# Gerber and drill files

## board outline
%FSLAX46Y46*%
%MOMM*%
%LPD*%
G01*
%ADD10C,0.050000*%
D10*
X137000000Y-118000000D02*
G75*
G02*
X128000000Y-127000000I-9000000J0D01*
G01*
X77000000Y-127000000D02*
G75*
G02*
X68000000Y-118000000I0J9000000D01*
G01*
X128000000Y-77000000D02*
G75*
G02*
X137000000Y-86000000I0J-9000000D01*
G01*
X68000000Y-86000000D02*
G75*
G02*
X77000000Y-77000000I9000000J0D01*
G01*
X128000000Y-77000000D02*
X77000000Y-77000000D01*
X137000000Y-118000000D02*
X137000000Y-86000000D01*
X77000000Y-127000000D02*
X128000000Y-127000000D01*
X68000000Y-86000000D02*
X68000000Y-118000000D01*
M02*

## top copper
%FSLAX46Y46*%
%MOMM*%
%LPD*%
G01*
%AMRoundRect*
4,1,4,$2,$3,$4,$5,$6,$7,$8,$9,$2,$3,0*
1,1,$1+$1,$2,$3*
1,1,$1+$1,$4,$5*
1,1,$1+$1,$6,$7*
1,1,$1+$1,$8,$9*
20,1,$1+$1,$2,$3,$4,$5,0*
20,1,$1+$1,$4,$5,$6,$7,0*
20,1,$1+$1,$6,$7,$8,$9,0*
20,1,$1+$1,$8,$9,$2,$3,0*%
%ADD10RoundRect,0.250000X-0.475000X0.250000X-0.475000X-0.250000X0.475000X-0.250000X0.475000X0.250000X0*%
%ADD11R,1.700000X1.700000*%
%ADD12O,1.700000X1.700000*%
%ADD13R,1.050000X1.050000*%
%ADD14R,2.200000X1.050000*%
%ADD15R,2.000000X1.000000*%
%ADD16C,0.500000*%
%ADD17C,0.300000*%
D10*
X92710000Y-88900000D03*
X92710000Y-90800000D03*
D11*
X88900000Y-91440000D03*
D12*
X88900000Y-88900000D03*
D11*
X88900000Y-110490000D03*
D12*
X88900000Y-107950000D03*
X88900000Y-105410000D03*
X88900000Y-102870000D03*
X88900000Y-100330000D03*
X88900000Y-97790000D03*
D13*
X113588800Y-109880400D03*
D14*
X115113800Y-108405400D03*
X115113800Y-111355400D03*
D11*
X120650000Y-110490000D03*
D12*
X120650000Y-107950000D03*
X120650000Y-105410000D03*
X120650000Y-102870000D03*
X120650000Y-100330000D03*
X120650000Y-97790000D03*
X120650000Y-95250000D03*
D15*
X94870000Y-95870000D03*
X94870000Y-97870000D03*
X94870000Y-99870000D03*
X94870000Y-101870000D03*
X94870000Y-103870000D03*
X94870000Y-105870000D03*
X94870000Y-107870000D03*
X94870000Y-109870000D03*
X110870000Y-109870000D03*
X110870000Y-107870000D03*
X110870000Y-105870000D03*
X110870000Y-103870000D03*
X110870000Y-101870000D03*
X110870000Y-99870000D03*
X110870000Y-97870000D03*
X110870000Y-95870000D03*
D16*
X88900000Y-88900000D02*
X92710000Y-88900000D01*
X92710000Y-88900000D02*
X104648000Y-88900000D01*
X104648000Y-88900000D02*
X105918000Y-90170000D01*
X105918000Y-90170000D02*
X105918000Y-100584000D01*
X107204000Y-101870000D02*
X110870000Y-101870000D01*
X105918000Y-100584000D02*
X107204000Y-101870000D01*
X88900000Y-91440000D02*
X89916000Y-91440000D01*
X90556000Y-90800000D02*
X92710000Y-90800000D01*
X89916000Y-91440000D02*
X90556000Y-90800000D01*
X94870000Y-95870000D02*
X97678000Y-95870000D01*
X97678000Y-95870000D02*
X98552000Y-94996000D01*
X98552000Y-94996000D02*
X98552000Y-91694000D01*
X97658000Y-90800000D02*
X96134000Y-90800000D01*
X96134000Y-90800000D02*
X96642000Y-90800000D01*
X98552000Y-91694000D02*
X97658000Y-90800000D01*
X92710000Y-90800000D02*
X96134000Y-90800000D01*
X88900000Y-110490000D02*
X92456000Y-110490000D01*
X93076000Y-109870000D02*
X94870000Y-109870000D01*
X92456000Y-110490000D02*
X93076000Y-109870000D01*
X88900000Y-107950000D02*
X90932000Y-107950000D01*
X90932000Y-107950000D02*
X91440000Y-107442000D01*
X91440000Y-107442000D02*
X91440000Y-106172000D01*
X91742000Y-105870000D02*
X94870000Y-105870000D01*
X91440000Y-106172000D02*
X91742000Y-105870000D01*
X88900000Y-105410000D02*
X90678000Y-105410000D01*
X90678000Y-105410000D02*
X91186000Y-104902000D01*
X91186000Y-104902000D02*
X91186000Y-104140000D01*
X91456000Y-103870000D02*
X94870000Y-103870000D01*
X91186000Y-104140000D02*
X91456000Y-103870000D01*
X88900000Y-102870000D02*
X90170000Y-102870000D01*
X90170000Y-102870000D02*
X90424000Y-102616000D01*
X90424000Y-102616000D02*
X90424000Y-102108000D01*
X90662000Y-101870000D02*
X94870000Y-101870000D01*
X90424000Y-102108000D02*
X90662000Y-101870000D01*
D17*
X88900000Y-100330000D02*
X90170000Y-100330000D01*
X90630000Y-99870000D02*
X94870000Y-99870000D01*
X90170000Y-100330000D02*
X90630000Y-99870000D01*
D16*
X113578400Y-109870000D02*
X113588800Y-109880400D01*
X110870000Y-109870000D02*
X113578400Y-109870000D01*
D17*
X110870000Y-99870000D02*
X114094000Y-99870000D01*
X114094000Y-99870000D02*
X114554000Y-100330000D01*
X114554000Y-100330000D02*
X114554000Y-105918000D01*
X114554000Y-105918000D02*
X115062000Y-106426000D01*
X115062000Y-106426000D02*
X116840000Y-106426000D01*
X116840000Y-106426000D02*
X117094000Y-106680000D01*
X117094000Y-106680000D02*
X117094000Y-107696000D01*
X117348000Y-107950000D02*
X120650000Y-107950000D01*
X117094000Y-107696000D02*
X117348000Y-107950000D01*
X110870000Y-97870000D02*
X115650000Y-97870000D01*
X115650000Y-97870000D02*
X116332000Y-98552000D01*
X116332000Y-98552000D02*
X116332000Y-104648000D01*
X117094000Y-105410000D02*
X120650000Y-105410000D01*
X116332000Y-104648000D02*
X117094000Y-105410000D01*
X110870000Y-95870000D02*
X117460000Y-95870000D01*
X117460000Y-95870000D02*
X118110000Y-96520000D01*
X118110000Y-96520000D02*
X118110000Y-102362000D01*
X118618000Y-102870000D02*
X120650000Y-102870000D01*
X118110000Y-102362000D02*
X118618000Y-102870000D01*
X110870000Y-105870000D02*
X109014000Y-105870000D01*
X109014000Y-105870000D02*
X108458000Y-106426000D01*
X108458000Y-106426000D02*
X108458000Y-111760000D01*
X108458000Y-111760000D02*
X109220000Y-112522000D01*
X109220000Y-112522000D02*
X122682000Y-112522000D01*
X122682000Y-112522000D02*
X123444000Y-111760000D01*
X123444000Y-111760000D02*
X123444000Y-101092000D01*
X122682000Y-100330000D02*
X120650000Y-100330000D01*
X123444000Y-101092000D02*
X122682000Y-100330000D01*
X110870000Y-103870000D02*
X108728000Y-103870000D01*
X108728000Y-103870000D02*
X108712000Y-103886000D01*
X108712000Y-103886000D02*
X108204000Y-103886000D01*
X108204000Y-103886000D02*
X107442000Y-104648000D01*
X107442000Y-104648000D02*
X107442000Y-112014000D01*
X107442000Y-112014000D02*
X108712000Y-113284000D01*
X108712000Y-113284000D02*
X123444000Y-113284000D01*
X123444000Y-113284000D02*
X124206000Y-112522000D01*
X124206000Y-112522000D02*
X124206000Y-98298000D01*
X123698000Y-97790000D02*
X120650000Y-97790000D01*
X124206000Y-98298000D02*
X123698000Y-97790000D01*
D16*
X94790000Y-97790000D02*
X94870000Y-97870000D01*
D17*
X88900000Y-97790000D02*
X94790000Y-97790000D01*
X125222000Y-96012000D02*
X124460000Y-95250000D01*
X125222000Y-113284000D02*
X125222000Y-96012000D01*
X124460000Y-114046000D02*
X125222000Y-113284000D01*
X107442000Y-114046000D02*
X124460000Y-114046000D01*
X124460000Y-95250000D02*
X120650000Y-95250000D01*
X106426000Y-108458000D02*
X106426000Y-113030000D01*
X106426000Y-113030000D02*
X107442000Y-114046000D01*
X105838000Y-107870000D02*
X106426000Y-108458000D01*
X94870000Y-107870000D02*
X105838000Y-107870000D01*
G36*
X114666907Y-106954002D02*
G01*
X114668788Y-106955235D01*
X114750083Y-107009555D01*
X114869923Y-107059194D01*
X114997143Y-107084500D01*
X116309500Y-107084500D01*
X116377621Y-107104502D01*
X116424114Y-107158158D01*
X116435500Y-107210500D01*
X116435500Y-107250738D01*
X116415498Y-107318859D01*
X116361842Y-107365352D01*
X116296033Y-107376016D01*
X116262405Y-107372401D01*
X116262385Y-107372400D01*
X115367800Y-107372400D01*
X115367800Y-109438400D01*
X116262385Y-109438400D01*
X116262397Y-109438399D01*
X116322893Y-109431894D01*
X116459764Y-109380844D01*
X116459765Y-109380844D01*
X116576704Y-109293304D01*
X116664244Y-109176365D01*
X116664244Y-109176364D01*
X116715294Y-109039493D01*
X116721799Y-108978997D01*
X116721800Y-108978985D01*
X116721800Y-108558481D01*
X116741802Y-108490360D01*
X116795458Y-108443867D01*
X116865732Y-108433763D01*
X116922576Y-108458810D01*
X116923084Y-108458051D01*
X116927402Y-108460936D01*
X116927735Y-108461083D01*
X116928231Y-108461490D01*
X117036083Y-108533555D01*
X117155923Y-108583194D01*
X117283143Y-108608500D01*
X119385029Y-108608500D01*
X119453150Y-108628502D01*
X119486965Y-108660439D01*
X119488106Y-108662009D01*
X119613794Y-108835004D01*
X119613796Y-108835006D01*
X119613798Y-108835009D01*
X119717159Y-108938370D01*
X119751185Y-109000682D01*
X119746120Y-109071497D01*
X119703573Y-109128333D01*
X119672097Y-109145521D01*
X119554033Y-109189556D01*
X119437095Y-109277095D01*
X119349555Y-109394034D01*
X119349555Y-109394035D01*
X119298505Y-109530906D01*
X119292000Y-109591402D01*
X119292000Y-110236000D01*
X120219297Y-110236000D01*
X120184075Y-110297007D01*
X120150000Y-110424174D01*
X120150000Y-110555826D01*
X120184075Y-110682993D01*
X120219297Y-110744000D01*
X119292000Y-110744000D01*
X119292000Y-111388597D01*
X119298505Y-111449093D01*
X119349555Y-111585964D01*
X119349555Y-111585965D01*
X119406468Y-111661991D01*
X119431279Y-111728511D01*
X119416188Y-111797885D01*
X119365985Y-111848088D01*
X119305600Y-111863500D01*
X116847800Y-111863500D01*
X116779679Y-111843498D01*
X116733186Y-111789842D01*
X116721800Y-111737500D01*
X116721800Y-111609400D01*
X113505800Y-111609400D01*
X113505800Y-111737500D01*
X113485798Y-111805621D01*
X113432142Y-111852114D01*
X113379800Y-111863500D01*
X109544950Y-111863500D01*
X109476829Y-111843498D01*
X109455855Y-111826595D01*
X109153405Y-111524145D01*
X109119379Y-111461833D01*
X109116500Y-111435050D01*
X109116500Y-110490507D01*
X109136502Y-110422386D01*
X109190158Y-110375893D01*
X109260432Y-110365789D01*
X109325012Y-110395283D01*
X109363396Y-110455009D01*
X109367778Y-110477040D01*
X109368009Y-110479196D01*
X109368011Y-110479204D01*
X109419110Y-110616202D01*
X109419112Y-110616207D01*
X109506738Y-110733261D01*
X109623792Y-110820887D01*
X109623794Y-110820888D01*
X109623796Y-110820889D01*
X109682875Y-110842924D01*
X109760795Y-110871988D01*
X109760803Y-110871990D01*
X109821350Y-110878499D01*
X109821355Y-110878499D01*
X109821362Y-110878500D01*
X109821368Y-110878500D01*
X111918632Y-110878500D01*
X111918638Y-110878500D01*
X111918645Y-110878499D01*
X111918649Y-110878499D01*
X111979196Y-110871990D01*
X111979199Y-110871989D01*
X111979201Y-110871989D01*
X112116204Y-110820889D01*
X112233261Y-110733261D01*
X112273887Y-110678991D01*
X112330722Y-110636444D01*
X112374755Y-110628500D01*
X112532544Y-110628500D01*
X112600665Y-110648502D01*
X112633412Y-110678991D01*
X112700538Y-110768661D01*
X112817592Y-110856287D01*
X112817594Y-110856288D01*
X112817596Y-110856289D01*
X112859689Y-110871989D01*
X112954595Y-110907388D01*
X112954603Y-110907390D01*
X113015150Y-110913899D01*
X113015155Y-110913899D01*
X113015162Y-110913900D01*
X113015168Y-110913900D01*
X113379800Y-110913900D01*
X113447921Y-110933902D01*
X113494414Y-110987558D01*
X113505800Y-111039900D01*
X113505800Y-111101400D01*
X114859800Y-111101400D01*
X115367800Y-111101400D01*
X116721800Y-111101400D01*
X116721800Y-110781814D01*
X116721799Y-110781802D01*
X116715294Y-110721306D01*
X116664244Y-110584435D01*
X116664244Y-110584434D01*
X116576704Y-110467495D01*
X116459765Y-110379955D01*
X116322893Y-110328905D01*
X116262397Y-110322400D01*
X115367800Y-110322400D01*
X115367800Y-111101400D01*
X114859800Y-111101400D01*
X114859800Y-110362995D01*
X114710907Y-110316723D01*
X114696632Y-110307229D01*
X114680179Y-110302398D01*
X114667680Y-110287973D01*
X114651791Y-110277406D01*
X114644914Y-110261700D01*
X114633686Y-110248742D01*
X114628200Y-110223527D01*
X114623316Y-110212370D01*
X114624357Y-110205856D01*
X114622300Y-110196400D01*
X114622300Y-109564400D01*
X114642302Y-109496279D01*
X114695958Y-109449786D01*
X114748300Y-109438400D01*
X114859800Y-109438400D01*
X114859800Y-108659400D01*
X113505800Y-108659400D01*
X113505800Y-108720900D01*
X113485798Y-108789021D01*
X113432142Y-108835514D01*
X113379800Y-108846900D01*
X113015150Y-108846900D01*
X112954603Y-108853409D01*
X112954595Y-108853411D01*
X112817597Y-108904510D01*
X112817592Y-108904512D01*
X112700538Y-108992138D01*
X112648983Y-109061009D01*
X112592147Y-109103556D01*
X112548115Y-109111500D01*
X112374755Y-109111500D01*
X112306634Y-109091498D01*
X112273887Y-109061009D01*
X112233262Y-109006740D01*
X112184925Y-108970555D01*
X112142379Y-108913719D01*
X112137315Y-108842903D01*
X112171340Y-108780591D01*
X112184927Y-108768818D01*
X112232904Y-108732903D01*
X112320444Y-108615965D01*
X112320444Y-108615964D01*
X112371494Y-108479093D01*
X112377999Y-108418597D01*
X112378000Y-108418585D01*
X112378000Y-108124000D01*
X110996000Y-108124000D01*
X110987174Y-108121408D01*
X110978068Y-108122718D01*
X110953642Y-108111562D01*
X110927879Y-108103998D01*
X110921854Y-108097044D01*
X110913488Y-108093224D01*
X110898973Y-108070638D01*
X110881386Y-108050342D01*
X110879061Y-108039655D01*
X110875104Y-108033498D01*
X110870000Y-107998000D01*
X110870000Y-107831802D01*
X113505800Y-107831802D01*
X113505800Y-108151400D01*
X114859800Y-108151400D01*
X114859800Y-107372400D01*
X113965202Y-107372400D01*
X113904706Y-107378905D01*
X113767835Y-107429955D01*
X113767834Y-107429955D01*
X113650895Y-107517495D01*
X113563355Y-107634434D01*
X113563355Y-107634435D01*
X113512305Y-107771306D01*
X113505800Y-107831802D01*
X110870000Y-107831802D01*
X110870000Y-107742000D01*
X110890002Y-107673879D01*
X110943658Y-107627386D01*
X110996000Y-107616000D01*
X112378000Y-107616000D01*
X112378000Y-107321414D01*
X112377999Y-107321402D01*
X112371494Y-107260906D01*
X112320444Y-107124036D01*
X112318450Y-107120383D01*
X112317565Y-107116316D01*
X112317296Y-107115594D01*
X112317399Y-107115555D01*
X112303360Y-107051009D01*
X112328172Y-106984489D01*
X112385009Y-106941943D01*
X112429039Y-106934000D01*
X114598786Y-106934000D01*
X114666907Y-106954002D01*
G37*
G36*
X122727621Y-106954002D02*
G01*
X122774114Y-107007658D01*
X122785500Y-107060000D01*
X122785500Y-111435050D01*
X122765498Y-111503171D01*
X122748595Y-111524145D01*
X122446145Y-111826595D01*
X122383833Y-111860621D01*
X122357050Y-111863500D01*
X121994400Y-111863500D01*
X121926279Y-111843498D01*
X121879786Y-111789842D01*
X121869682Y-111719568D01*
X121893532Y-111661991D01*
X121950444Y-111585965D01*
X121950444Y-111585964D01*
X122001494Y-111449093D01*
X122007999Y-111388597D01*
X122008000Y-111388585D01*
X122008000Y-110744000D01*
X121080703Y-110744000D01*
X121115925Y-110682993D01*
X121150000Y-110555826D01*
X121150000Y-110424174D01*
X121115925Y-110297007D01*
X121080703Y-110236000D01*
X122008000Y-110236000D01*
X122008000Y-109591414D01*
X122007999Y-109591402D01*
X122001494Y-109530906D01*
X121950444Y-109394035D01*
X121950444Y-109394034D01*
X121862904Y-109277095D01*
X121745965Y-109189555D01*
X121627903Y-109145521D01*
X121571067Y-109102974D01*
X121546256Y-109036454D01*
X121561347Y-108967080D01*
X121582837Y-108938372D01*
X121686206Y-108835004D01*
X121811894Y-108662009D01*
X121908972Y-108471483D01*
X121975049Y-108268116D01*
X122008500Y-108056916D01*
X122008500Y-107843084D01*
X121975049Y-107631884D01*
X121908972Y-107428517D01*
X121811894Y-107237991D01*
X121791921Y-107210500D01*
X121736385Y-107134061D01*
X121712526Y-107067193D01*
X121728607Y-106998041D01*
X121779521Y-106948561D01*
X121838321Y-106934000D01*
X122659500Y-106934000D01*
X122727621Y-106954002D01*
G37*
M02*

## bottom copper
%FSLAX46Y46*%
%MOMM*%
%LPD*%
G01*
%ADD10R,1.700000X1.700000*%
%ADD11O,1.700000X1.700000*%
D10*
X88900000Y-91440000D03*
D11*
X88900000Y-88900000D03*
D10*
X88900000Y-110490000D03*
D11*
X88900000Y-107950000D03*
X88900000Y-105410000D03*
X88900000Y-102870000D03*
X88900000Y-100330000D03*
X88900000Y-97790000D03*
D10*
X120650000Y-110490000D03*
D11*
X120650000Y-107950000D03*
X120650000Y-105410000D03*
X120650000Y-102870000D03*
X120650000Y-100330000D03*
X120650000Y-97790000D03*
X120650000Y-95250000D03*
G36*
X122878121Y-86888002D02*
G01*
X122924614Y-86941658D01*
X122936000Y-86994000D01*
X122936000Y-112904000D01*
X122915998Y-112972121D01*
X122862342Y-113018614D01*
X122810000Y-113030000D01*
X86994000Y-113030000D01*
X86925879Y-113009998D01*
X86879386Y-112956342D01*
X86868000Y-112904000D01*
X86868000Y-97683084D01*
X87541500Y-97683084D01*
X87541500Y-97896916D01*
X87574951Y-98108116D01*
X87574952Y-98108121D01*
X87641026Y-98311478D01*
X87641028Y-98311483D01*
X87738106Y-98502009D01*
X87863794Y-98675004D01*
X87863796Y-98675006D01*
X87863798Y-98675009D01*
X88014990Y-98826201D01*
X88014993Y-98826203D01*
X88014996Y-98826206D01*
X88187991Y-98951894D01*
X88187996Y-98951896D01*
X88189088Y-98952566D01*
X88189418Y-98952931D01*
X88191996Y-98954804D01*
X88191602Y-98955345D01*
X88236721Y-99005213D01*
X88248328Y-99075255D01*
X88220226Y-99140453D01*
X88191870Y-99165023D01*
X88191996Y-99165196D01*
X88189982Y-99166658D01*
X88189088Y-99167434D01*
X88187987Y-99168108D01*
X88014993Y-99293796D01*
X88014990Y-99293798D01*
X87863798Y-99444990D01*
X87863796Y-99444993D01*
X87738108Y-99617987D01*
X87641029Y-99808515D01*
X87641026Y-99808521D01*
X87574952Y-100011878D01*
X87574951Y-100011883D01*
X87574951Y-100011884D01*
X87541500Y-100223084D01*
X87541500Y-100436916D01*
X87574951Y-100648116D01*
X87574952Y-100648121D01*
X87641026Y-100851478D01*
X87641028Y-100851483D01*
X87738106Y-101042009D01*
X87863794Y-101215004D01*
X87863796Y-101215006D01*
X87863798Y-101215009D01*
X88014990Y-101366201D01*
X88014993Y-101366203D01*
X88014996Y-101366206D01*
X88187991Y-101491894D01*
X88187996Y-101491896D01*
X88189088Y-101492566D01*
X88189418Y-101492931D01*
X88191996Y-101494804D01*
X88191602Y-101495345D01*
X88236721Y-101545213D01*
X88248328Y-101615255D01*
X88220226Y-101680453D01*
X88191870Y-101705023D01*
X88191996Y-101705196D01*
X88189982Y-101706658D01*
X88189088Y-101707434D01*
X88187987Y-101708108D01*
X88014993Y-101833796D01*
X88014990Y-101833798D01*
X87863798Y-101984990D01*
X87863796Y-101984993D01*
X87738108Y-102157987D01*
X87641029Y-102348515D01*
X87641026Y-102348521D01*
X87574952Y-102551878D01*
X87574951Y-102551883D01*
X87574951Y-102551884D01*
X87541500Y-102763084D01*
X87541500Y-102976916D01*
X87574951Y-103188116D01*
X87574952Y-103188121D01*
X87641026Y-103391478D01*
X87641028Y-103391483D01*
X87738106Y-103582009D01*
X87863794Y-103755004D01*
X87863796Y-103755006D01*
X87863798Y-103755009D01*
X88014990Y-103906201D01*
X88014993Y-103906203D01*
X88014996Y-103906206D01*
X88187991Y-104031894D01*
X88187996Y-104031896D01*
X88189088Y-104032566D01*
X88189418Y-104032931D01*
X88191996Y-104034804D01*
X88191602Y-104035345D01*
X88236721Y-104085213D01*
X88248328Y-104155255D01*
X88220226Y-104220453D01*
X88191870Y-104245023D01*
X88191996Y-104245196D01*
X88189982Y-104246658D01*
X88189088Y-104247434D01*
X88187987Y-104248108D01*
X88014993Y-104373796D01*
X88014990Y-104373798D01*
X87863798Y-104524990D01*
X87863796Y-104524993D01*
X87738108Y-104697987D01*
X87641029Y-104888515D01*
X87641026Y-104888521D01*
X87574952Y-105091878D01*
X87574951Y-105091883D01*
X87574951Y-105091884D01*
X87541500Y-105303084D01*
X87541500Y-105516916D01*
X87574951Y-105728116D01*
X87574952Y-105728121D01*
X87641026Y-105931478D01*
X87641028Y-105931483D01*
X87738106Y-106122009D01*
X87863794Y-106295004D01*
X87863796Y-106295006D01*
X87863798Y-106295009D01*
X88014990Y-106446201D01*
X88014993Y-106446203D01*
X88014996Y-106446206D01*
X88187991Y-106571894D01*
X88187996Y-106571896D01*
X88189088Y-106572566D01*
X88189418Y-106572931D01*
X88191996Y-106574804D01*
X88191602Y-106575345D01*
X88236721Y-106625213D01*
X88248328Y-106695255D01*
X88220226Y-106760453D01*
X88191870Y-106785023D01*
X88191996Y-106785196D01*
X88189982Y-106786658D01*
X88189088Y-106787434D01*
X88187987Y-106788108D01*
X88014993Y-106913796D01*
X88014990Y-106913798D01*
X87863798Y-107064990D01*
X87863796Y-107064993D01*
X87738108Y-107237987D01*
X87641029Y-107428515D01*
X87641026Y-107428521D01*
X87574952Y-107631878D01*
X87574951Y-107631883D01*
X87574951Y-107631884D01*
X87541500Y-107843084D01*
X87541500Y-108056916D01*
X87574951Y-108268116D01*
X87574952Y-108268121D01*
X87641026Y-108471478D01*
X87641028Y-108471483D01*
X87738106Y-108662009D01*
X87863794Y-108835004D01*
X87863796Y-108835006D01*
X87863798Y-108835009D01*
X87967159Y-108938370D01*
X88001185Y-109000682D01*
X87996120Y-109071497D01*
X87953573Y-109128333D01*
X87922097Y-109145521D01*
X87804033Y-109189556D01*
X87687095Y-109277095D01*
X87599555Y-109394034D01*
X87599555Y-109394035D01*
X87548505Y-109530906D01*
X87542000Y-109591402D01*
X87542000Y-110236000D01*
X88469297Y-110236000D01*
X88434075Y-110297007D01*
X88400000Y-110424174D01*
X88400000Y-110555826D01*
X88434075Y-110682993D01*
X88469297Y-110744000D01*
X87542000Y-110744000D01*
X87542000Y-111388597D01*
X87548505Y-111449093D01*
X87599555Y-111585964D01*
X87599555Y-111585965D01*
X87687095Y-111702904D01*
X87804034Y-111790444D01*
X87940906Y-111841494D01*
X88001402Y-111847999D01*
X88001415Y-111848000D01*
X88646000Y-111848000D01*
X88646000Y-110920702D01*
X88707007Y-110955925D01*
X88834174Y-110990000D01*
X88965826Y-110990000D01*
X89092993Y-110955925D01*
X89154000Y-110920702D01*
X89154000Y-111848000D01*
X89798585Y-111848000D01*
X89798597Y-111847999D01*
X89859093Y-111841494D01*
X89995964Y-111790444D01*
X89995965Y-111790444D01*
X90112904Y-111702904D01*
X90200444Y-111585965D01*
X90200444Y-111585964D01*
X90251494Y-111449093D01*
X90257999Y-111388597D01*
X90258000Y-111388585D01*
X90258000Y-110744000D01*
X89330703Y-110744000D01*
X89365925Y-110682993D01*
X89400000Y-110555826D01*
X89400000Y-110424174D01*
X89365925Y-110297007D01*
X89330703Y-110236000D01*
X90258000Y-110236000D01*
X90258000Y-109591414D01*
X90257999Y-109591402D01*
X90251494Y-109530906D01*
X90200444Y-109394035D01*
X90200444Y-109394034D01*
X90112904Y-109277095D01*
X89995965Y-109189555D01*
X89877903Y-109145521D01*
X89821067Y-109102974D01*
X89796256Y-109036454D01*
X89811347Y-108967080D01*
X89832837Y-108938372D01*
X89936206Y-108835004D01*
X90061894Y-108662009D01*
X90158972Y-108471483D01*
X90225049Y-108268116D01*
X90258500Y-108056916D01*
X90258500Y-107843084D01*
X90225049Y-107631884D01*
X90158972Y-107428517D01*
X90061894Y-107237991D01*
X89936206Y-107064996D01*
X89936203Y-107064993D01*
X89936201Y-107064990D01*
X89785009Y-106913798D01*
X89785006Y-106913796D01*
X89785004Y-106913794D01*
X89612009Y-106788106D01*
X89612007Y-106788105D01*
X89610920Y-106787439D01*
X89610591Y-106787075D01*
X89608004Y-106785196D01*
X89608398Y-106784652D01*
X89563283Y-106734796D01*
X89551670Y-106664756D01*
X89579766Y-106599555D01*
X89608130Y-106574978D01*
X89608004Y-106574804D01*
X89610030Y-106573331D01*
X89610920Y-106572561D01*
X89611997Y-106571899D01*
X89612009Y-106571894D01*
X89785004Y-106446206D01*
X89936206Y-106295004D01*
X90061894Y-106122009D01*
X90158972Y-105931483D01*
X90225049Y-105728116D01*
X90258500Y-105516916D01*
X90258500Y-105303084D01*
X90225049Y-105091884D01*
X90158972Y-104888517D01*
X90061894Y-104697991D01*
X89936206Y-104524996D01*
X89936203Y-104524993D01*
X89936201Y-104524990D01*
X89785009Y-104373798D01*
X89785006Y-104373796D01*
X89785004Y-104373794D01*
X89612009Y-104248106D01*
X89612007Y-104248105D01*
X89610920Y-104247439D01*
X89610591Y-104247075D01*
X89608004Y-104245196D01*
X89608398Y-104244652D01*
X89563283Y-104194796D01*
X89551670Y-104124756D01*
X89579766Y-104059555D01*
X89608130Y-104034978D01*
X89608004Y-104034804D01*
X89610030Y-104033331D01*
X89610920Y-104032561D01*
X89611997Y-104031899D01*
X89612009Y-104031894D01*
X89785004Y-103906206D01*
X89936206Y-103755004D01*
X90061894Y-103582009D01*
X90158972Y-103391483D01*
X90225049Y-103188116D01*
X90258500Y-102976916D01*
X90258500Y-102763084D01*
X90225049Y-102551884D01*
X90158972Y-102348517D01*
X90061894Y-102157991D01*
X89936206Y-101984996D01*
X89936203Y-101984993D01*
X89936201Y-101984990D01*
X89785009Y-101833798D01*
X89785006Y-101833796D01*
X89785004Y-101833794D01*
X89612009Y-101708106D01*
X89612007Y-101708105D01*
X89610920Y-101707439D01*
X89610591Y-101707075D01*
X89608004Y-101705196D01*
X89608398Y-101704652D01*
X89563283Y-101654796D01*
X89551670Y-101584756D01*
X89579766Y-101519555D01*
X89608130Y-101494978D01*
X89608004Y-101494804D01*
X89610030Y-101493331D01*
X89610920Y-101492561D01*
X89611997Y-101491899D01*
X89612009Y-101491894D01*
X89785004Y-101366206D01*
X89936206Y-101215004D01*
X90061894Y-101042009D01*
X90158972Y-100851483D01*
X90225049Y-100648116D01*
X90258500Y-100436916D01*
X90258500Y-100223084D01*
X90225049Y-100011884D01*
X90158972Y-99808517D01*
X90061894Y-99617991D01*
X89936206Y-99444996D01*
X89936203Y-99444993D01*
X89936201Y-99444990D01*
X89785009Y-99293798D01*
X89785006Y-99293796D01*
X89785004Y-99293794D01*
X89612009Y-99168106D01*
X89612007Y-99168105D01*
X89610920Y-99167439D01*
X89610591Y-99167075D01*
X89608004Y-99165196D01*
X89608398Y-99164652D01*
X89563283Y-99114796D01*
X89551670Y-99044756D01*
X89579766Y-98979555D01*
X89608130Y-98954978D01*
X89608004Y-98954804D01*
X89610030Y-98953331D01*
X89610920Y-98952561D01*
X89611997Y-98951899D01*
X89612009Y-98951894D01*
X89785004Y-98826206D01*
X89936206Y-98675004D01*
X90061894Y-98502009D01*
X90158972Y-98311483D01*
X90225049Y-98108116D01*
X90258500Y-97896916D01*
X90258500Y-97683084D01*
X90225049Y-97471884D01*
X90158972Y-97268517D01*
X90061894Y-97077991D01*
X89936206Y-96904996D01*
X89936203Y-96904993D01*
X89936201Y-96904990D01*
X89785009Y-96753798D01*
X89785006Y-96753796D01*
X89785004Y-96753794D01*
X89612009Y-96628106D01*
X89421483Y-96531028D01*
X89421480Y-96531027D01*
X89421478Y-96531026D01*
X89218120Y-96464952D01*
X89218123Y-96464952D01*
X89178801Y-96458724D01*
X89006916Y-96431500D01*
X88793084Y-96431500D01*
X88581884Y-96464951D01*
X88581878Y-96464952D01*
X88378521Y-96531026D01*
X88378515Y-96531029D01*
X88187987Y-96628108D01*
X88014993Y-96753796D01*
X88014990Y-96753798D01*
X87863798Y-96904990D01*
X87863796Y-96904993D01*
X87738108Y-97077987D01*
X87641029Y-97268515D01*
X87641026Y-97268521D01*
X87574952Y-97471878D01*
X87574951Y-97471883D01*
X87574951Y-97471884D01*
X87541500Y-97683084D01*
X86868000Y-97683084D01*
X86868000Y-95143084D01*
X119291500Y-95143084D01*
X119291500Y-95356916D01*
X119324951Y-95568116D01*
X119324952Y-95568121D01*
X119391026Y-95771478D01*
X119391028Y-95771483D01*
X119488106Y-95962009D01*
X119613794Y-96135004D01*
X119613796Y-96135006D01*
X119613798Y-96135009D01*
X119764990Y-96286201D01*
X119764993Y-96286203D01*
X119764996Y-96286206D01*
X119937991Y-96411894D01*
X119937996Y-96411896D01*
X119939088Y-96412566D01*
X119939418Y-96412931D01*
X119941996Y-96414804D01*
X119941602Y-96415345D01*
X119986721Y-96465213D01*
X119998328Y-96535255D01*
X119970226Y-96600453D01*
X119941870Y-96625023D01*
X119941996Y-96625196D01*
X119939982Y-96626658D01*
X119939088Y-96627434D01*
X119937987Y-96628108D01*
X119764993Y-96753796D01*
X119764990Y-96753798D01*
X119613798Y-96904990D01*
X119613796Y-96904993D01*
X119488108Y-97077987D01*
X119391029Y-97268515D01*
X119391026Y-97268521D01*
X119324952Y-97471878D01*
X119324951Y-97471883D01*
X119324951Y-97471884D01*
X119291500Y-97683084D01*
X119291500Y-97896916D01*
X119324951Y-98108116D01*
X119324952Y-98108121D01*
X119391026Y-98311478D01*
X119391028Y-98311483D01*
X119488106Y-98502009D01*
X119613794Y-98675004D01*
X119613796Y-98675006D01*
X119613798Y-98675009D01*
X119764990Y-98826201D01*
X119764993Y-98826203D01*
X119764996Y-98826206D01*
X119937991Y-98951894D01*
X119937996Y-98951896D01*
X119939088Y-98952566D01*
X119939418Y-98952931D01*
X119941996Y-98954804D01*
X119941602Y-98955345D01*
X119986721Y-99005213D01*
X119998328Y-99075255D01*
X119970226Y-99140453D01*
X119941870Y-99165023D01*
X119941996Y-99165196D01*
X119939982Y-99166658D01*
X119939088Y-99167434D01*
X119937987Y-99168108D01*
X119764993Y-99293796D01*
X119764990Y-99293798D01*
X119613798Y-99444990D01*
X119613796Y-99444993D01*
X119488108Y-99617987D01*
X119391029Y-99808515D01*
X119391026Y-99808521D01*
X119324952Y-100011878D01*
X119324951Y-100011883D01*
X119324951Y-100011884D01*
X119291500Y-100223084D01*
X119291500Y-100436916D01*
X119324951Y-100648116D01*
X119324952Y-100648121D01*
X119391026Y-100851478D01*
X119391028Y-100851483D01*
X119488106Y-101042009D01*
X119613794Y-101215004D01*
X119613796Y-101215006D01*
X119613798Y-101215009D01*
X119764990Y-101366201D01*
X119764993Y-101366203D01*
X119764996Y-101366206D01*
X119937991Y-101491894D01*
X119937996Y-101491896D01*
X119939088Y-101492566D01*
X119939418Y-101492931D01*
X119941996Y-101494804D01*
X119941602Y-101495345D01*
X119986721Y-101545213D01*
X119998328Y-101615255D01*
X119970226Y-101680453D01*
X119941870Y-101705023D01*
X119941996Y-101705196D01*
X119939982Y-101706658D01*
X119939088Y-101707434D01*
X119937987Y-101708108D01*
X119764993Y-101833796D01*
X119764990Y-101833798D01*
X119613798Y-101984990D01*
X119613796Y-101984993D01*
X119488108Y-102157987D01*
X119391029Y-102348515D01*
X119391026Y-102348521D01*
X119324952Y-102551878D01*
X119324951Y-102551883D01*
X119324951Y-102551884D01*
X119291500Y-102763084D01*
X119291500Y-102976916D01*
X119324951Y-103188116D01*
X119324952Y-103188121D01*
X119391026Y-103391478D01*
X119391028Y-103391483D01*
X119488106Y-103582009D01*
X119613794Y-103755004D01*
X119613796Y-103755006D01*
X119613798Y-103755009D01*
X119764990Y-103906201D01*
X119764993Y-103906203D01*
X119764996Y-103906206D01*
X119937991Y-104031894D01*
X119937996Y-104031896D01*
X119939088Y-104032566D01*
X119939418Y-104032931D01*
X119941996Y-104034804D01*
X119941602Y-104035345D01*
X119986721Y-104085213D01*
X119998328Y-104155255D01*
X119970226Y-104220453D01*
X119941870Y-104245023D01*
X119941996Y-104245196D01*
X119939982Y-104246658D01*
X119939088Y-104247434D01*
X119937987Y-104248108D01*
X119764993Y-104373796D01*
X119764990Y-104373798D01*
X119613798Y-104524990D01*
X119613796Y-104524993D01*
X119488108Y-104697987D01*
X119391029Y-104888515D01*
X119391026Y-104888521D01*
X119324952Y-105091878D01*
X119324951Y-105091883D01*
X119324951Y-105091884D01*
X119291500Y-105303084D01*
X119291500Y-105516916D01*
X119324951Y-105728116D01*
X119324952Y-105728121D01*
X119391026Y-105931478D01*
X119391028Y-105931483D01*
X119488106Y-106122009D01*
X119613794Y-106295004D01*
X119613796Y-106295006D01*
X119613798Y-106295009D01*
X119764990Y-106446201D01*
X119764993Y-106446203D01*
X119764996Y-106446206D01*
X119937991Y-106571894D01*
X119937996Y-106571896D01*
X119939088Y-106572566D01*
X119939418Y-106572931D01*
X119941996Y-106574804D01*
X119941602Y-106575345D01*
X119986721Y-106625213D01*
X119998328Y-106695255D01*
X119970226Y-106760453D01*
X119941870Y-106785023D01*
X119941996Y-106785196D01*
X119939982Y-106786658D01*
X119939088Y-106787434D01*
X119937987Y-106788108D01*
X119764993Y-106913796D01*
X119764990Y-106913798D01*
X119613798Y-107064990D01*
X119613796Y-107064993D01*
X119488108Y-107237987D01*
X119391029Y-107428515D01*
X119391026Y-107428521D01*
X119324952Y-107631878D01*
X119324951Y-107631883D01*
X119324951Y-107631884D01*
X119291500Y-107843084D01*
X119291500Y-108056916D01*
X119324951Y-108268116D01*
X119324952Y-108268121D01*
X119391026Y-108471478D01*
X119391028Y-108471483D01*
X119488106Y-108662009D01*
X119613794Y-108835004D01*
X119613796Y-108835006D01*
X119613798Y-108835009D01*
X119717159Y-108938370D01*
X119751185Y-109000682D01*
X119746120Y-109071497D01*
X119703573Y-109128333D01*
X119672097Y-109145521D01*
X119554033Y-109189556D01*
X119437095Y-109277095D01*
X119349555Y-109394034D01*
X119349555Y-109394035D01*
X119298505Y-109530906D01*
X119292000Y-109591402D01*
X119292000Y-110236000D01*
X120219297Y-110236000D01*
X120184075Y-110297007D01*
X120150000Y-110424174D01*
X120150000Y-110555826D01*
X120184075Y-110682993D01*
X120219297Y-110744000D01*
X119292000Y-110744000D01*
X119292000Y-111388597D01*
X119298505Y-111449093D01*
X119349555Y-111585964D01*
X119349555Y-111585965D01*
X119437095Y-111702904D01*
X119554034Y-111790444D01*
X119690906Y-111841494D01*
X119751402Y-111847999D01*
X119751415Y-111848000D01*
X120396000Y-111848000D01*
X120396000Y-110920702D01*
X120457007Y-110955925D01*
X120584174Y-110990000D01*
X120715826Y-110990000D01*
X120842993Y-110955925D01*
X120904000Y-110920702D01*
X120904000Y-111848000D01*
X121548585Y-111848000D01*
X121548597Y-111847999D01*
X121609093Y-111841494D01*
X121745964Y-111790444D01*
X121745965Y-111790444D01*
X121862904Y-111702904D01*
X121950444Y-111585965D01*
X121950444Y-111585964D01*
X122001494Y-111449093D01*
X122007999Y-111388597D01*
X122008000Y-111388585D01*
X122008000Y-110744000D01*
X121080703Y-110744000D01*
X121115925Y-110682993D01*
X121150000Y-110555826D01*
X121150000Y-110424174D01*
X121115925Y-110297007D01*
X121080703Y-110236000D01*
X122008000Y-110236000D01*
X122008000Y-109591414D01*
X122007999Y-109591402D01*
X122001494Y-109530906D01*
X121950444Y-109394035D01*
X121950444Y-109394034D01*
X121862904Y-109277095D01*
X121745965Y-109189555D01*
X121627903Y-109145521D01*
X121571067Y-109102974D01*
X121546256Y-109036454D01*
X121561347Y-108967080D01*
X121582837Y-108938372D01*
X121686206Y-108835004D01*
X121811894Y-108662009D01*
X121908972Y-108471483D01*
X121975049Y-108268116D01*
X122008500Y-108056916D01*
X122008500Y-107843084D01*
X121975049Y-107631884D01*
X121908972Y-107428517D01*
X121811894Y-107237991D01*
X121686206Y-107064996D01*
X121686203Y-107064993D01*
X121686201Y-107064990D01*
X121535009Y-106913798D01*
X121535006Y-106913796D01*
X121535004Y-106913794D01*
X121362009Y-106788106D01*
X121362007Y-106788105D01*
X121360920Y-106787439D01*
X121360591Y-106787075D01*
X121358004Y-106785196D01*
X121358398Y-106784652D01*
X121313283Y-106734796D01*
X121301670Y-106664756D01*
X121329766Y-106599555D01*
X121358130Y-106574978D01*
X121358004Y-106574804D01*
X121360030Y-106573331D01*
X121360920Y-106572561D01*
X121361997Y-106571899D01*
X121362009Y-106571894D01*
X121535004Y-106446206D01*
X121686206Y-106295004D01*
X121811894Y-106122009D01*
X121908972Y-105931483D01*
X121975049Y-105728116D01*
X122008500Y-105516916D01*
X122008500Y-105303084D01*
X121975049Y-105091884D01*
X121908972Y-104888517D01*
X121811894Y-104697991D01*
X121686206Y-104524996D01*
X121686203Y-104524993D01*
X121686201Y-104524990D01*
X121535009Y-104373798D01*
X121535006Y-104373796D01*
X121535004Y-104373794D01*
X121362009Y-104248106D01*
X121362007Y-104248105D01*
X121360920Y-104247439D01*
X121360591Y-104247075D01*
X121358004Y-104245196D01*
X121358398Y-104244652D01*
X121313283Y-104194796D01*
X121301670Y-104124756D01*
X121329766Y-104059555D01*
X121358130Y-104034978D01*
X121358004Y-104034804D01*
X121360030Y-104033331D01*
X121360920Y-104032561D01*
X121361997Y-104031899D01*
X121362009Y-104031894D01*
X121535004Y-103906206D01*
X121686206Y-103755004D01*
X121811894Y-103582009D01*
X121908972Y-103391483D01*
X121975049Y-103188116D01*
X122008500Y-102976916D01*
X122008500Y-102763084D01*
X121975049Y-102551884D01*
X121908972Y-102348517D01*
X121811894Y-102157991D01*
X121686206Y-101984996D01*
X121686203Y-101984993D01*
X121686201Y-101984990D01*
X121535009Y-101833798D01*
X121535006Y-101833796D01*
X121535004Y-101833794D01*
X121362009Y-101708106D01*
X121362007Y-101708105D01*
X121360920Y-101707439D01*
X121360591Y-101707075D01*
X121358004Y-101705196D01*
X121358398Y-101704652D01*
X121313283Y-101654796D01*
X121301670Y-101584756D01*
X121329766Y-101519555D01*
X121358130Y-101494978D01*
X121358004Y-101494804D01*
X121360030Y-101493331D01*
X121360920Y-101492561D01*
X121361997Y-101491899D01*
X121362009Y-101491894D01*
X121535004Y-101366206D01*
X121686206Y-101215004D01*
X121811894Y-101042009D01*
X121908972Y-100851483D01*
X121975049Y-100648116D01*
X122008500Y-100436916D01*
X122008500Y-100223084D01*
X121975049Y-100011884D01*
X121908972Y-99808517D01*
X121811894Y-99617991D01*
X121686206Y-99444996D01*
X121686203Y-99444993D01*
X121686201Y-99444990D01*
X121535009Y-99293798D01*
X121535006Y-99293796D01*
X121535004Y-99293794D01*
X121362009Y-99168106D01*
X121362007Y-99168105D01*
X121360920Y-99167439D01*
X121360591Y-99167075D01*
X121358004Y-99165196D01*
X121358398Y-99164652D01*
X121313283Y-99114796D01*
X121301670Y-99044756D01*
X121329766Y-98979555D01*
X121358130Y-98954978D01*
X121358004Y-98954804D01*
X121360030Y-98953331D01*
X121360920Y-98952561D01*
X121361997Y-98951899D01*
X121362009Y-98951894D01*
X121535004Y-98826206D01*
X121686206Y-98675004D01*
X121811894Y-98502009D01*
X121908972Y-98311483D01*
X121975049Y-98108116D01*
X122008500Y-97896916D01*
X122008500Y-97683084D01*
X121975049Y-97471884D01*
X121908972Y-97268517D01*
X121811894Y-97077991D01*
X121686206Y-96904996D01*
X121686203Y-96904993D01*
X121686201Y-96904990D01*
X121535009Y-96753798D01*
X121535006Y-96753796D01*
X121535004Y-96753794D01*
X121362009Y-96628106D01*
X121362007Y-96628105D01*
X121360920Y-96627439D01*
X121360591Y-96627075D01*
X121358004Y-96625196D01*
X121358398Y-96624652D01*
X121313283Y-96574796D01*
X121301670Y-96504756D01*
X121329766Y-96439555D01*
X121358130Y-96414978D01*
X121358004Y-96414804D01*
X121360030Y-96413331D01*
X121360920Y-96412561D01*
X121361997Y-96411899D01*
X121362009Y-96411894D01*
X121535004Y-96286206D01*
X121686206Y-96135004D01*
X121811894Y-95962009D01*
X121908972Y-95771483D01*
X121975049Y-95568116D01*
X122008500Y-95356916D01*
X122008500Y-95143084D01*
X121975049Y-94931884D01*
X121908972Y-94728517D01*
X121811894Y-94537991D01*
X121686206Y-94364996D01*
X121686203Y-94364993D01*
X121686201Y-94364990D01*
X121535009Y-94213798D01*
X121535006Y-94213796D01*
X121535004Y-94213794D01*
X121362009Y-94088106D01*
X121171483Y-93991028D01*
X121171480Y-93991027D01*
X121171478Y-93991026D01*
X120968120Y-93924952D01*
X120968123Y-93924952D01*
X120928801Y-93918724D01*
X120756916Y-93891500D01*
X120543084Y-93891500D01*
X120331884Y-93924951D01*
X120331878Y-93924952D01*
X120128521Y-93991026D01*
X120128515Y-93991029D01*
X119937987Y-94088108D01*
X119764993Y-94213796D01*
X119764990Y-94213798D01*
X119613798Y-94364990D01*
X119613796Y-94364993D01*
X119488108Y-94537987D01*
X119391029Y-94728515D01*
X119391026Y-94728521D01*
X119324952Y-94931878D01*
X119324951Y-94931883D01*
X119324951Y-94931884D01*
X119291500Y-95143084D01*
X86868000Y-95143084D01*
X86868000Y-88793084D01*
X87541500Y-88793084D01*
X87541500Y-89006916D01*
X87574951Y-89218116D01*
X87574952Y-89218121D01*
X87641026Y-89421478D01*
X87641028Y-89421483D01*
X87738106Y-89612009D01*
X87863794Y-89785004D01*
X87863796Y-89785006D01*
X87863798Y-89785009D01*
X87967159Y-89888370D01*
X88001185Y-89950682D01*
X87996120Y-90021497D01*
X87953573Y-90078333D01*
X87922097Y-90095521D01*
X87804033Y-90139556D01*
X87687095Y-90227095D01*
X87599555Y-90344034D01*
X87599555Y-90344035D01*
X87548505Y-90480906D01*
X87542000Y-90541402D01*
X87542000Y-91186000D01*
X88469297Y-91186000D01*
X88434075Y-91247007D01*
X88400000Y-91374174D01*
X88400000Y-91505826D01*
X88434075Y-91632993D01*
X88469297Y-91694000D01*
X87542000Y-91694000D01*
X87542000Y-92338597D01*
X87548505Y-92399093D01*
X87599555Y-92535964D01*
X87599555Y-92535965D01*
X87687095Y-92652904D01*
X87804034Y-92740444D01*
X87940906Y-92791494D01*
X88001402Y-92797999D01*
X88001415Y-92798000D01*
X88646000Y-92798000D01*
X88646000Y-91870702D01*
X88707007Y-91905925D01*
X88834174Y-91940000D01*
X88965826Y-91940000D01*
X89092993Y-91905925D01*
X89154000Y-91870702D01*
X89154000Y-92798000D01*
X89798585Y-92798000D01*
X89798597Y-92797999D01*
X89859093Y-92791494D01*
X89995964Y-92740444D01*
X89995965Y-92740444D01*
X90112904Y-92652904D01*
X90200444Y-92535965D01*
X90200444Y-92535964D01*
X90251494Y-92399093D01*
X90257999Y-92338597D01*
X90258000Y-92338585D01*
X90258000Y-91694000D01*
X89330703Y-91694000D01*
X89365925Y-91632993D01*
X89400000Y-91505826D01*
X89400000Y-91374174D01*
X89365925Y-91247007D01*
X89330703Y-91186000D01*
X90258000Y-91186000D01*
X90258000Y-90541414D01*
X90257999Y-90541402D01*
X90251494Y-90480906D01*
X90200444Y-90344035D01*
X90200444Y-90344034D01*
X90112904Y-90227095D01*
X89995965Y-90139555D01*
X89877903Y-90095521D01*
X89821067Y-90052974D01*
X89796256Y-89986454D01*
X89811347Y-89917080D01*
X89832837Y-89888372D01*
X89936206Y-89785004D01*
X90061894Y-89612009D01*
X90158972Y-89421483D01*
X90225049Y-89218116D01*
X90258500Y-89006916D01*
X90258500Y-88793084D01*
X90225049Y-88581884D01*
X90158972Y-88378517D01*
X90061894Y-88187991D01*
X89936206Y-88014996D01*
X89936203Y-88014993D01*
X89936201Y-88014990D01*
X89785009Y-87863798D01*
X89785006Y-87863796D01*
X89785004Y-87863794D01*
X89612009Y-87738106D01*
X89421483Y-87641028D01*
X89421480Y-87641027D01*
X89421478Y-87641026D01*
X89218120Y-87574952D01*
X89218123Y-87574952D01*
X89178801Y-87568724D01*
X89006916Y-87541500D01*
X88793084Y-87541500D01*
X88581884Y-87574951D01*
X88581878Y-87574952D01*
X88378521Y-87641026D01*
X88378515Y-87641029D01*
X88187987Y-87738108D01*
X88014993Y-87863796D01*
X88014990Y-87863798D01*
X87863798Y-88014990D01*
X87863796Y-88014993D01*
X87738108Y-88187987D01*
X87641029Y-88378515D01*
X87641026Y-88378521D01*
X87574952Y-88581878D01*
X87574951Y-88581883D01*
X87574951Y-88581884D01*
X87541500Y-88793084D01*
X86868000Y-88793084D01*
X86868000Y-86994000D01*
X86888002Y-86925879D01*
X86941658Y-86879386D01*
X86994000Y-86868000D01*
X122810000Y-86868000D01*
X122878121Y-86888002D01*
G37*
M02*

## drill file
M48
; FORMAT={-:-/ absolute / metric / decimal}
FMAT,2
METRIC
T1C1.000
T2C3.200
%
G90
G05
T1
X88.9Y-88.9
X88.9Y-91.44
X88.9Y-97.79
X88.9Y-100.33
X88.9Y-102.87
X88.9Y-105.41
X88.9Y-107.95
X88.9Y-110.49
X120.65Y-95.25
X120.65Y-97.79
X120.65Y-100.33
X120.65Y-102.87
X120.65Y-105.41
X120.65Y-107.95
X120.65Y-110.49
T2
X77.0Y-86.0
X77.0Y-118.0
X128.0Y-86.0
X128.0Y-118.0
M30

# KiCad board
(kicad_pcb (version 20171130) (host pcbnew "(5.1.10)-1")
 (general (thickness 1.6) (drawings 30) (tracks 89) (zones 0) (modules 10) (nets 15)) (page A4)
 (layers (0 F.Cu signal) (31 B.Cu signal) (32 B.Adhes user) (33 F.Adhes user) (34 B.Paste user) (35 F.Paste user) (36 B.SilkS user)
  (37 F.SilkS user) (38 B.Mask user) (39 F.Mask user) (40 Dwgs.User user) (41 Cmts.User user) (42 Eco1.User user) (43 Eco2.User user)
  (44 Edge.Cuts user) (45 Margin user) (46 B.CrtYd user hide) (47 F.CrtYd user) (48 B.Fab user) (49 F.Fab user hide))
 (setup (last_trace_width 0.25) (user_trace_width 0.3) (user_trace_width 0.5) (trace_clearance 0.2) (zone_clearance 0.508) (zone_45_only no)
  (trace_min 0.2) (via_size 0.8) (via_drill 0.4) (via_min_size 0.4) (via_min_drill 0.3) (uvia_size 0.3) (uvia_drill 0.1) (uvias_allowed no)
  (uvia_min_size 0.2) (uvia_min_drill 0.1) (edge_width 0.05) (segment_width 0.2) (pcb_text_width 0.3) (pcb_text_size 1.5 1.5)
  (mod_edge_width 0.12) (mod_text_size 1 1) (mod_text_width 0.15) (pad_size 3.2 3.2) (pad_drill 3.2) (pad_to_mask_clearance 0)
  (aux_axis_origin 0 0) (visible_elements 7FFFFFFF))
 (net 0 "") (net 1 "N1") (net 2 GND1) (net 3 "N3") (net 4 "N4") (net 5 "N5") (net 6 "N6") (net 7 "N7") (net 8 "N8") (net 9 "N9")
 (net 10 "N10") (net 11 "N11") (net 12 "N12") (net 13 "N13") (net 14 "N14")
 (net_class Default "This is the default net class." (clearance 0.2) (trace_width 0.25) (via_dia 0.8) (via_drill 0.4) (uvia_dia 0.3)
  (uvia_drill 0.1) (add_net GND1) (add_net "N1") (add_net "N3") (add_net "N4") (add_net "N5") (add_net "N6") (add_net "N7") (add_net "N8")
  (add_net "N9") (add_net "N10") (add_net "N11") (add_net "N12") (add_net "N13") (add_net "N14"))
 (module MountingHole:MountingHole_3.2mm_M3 (layer F.Cu) (at 77 86)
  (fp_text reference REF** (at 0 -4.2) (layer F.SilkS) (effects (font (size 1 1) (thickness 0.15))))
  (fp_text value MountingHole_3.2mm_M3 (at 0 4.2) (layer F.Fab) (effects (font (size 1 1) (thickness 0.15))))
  (pad 1 np_thru_hole circle (at 0 0) (size 3.2 3.2) (drill 3.2) (layers *.Cu *.Mask)))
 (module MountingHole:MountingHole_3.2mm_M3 (layer F.Cu) (at 128 86)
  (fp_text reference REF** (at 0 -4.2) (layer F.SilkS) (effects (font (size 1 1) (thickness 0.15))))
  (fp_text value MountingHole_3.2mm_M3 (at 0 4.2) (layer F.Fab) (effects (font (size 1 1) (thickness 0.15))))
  (pad 1 np_thru_hole circle (at 0 0) (size 3.2 3.2) (drill 3.2) (layers *.Cu *.Mask)))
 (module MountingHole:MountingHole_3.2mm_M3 (layer F.Cu) (at 128 118)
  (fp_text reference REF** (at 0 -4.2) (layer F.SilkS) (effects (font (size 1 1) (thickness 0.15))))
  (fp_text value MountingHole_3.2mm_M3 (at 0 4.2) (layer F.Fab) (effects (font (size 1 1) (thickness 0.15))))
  (pad 1 np_thru_hole circle (at 0 0) (size 3.2 3.2) (drill 3.2) (layers *.Cu *.Mask)))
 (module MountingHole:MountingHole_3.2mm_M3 (layer F.Cu) (at 77 118)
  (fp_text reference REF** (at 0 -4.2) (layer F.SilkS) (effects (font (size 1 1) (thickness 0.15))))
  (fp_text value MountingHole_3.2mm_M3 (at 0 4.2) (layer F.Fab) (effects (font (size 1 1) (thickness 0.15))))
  (pad 1 np_thru_hole circle (at 0 0) (size 3.2 3.2) (drill 3.2) (layers *.Cu *.Mask)))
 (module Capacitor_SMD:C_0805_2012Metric (layer F.Cu) (at 92.71 89.85 270)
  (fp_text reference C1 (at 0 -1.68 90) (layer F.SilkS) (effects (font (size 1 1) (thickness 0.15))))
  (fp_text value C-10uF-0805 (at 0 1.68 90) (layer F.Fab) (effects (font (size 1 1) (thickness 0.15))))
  (pad 1 smd roundrect (at -0.95 0 270) (size 1 1.45) (layers F.Cu F.Paste F.Mask) (roundrect_rratio 0.25) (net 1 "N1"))
  (pad 2 smd roundrect (at 0.95 0 270) (size 1 1.45) (layers F.Cu F.Paste F.Mask) (roundrect_rratio 0.25) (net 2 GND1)))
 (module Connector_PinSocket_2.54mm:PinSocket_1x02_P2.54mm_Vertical (layer F.Cu) (at 88.9 91.44 180)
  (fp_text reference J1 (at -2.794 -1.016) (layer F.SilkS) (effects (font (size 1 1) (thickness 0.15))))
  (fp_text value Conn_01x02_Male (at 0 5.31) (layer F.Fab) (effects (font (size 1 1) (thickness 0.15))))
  (pad 1 thru_hole rect (at 0 0 180) (size 1.7 1.7) (drill 1) (layers *.Cu *.Mask) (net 2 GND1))
  (pad 2 thru_hole oval (at 0 2.54 180) (size 1.7 1.7) (drill 1) (layers *.Cu *.Mask) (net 1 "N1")))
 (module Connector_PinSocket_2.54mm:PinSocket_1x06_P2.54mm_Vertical (layer F.Cu) (at 88.9 110.49 180)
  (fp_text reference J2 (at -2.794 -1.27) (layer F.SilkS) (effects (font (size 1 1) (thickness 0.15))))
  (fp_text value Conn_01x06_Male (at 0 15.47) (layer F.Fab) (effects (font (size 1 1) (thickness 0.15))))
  (pad 1 thru_hole rect (at 0 0 180) (size 1.7 1.7) (drill 1) (layers *.Cu *.Mask) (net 2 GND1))
  (pad 2 thru_hole oval (at 0 2.54 180) (size 1.7 1.7) (drill 1) (layers *.Cu *.Mask) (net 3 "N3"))
  (pad 3 thru_hole oval (at 0 5.08 180) (size 1.7 1.7) (drill 1) (layers *.Cu *.Mask) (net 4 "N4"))
  (pad 4 thru_hole oval (at 0 7.62 180) (size 1.7 1.7) (drill 1) (layers *.Cu *.Mask) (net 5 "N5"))
  (pad 5 thru_hole oval (at 0 10.16 180) (size 1.7 1.7) (drill 1) (layers *.Cu *.Mask) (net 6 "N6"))
  (pad 6 thru_hole oval (at 0 12.7 180) (size 1.7 1.7) (drill 1) (layers *.Cu *.Mask) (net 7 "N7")))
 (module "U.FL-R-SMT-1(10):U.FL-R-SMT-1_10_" (layer F.Cu) (at 115.1138 109.8804 90)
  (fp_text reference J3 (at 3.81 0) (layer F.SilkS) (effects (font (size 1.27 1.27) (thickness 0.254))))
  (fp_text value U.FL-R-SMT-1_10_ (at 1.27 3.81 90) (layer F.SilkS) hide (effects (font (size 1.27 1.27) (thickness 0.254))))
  (pad 3 smd rect (at 0 -1.525 180) (size 1.05 1.05) (layers F.Cu F.Paste F.Mask) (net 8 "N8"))
  (pad 2 smd rect (at 1.475 0 90) (size 1.05 2.2) (layers F.Cu F.Paste F.Mask) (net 2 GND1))
  (pad 1 smd rect (at -1.475 0 90) (size 1.05 2.2) (layers F.Cu F.Paste F.Mask) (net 2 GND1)))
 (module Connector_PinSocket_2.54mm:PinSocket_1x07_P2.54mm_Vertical (layer F.Cu) (at 120.65 110.49 180)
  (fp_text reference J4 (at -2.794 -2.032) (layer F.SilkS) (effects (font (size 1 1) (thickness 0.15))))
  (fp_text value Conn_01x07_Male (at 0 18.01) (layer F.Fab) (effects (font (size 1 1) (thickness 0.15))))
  (pad 1 thru_hole rect (at 0 0 180) (size 1.7 1.7) (drill 1) (layers *.Cu *.Mask) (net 2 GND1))
  (pad 2 thru_hole oval (at 0 2.54 180) (size 1.7 1.7) (drill 1) (layers *.Cu *.Mask) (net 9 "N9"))
  (pad 3 thru_hole oval (at 0 5.08 180) (size 1.7 1.7) (drill 1) (layers *.Cu *.Mask) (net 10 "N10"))
  (pad 4 thru_hole oval (at 0 7.62 180) (size 1.7 1.7) (drill 1) (layers *.Cu *.Mask) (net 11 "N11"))
  (pad 5 thru_hole oval (at 0 10.16 180) (size 1.7 1.7) (drill 1) (layers *.Cu *.Mask) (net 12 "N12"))
  (pad 6 thru_hole oval (at 0 12.7 180) (size 1.7 1.7) (drill 1) (layers *.Cu *.Mask) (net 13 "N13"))
  (pad 7 thru_hole oval (at 0 15.24 180) (size 1.7 1.7) (drill 1) (layers *.Cu *.Mask) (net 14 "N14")))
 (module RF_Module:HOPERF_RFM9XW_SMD (layer F.Cu) (at 102.87 102.87)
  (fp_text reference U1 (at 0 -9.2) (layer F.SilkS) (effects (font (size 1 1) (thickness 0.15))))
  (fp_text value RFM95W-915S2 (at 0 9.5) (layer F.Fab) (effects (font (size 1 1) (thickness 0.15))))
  (pad 1 smd rect (at -8 -7) (size 2 1) (layers F.Cu F.Paste F.Mask) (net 2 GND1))
  (pad 2 smd rect (at -8 -5) (size 2 1) (layers F.Cu F.Paste F.Mask) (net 7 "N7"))
  (pad 3 smd rect (at -8 -3) (size 2 1) (layers F.Cu F.Paste F.Mask) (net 6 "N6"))
  (pad 4 smd rect (at -8 -1) (size 2 1) (layers F.Cu F.Paste F.Mask) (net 5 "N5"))
  (pad 5 smd rect (at -8 1) (size 2 1) (layers F.Cu F.Paste F.Mask) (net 4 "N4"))
  (pad 6 smd rect (at -8 3) (size 2 1) (layers F.Cu F.Paste F.Mask) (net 3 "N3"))
  (pad 7 smd rect (at -8 5) (size 2 1) (layers F.Cu F.Paste F.Mask) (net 14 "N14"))
  (pad 8 smd rect (at -8 7) (size 2 1) (layers F.Cu F.Paste F.Mask) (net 2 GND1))
  (pad 9 smd rect (at 8 7) (size 2 1) (layers F.Cu F.Paste F.Mask) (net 8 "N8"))
  (pad 10 smd rect (at 8 5) (size 2 1) (layers F.Cu F.Paste F.Mask) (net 2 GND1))
  (pad 11 smd rect (at 8 3) (size 2 1) (layers F.Cu F.Paste F.Mask) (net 12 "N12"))
  (pad 12 smd rect (at 8 1) (size 2 1) (layers F.Cu F.Paste F.Mask) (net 13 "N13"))
  (pad 13 smd rect (at 8 -1) (size 2 1) (layers F.Cu F.Paste F.Mask) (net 1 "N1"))
  (pad 14 smd rect (at 8 -3) (size 2 1) (layers F.Cu F.Paste F.Mask) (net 9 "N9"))
  (pad 15 smd rect (at 8 -5) (size 2 1) (layers F.Cu F.Paste F.Mask) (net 10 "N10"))
  (pad 16 smd rect (at 8 -7) (size 2 1) (layers F.Cu F.Paste F.Mask) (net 11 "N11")))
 (gr_arc (start 128 118) (end 128 127) (angle -90) (layer Edge.Cuts) (width 0.05))
 (gr_arc (start 77 118) (end 68 118) (angle -90) (layer Edge.Cuts) (width 0.05))
 (gr_arc (start 128 86) (end 137 86) (angle -90) (layer Edge.Cuts) (width 0.05))
 (gr_arc (start 77 86) (end 77 77) (angle -90) (layer Edge.Cuts) (width 0.05))
 (gr_line (start 128 77) (end 77 77) (layer Edge.Cuts) (width 0.05))
 (gr_line (start 137 118) (end 137 86) (layer Edge.Cuts) (width 0.05))
 (gr_line (start 77 127) (end 128 127) (layer Edge.Cuts) (width 0.05))
 (gr_line (start 68 86) (end 68 118) (layer Edge.Cuts) (width 0.05))
 (segment (start 88.9 88.9) (end 92.71 88.9) (width 0.5) (layer F.Cu) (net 1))
 (segment (start 92.71 88.9) (end 104.648 88.9) (width 0.5) (layer F.Cu) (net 1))
 (segment (start 104.648 88.9) (end 105.918 90.17) (width 0.5) (layer F.Cu) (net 1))
 (segment (start 105.918 90.17) (end 105.918 100.584) (width 0.5) (layer F.Cu) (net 1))
 (segment (start 107.204 101.87) (end 110.87 101.87) (width 0.5) (layer F.Cu) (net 1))
 (segment (start 105.918 100.584) (end 107.204 101.87) (width 0.5) (layer F.Cu) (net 1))
 (segment (start 88.9 91.44) (end 89.916 91.44) (width 0.5) (layer F.Cu) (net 2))
 (segment (start 90.556 90.8) (end 92.71 90.8) (width 0.5) (layer F.Cu) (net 2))
 (segment (start 89.916 91.44) (end 90.556 90.8) (width 0.5) (layer F.Cu) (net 2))
 (segment (start 94.87 95.87) (end 97.678 95.87) (width 0.5) (layer F.Cu) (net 2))
 (segment (start 97.678 95.87) (end 98.552 94.996) (width 0.5) (layer F.Cu) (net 2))
 (segment (start 98.552 94.996) (end 98.552 91.694) (width 0.5) (layer F.Cu) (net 2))
 (segment (start 97.658 90.8) (end 96.134 90.8) (width 0.5) (layer F.Cu) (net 2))
 (segment (start 96.134 90.8) (end 96.642 90.8) (width 0.5) (layer F.Cu) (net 2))
 (segment (start 98.552 91.694) (end 97.658 90.8) (width 0.5) (layer F.Cu) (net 2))
 (segment (start 92.71 90.8) (end 96.134 90.8) (width 0.5) (layer F.Cu) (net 2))
 (segment (start 88.9 110.49) (end 92.456 110.49) (width 0.5) (layer F.Cu) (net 2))
 (segment (start 93.076 109.87) (end 94.87 109.87) (width 0.5) (layer F.Cu) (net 2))
 (segment (start 92.456 110.49) (end 93.076 109.87) (width 0.5) (layer F.Cu) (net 2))
 (segment (start 88.9 107.95) (end 90.932 107.95) (width 0.5) (layer F.Cu) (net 3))
 (segment (start 90.932 107.95) (end 91.44 107.442) (width 0.5) (layer F.Cu) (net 3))
 (segment (start 91.44 107.442) (end 91.44 106.172) (width 0.5) (layer F.Cu) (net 3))
 (segment (start 91.742 105.87) (end 94.87 105.87) (width 0.5) (layer F.Cu) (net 3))
 (segment (start 91.44 106.172) (end 91.742 105.87) (width 0.5) (layer F.Cu) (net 3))
 (segment (start 88.9 105.41) (end 90.678 105.41) (width 0.5) (layer F.Cu) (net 4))
 (segment (start 90.678 105.41) (end 91.186 104.902) (width 0.5) (layer F.Cu) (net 4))
 (segment (start 91.186 104.902) (end 91.186 104.14) (width 0.5) (layer F.Cu) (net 4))
 (segment (start 91.456 103.87) (end 94.87 103.87) (width 0.5) (layer F.Cu) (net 4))
 (segment (start 91.186 104.14) (end 91.456 103.87) (width 0.5) (layer F.Cu) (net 4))
 (segment (start 88.9 102.87) (end 90.17 102.87) (width 0.5) (layer F.Cu) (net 5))
 (segment (start 90.17 102.87) (end 90.424 102.616) (width 0.5) (layer F.Cu) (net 5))
 (segment (start 90.424 102.616) (end 90.424 102.108) (width 0.5) (layer F.Cu) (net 5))
 (segment (start 90.662 101.87) (end 94.87 101.87) (width 0.5) (layer F.Cu) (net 5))
 (segment (start 90.424 102.108) (end 90.662 101.87) (width 0.5) (layer F.Cu) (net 5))
 (segment (start 88.9 100.33) (end 90.17 100.33) (width 0.3) (layer F.Cu) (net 6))
 (segment (start 90.63 99.87) (end 94.87 99.87) (width 0.3) (layer F.Cu) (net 6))
 (segment (start 90.17 100.33) (end 90.63 99.87) (width 0.3) (layer F.Cu) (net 6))
 (segment (start 113.5784 109.87) (end 113.5888 109.8804) (width 0.5) (layer F.Cu) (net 8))
 (segment (start 110.87 109.87) (end 113.5784 109.87) (width 0.5) (layer F.Cu) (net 8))
 (segment (start 110.87 99.87) (end 114.094 99.87) (width 0.3) (layer F.Cu) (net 9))
 (segment (start 114.094 99.87) (end 114.554 100.33) (width 0.3) (layer F.Cu) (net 9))
 (segment (start 114.554 100.33) (end 114.554 105.918) (width 0.3) (layer F.Cu) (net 9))
 (segment (start 114.554 105.918) (end 115.062 106.426) (width 0.3) (layer F.Cu) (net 9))
 (segment (start 115.062 106.426) (end 116.84 106.426) (width 0.3) (layer F.Cu) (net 9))
 (segment (start 116.84 106.426) (end 117.094 106.68) (width 0.3) (layer F.Cu) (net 9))
 (segment (start 117.094 106.68) (end 117.094 107.696) (width 0.3) (layer F.Cu) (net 9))
 (segment (start 117.348 107.95) (end 120.65 107.95) (width 0.3) (layer F.Cu) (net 9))
 (segment (start 117.094 107.696) (end 117.348 107.95) (width 0.3) (layer F.Cu) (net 9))
 (segment (start 110.87 97.87) (end 115.65 97.87) (width 0.3) (layer F.Cu) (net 10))
 (segment (start 115.65 97.87) (end 116.332 98.552) (width 0.3) (layer F.Cu) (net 10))
 (segment (start 116.332 98.552) (end 116.332 104.648) (width 0.3) (layer F.Cu) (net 10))
 (segment (start 117.094 105.41) (end 120.65 105.41) (width 0.3) (layer F.Cu) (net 10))
 (segment (start 116.332 104.648) (end 117.094 105.41) (width 0.3) (layer F.Cu) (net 10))
 (segment (start 110.87 95.87) (end 117.46 95.87) (width 0.3) (layer F.Cu) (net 11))
 (segment (start 117.46 95.87) (end 118.11 96.52) (width 0.3) (layer F.Cu) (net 11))
 (segment (start 118.11 96.52) (end 118.11 102.362) (width 0.3) (layer F.Cu) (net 11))
 (segment (start 118.618 102.87) (end 120.65 102.87) (width 0.3) (layer F.Cu) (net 11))
 (segment (start 118.11 102.362) (end 118.618 102.87) (width 0.3) (layer F.Cu) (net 11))
 (segment (start 110.87 105.87) (end 109.014 105.87) (width 0.3) (layer F.Cu) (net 12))
 (segment (start 109.014 105.87) (end 108.458 106.426) (width 0.3) (layer F.Cu) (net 12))
 (segment (start 108.458 106.426) (end 108.458 111.76) (width 0.3) (layer F.Cu) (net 12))
 (segment (start 108.458 111.76) (end 109.22 112.522) (width 0.3) (layer F.Cu) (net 12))
 (segment (start 109.22 112.522) (end 122.682 112.522) (width 0.3) (layer F.Cu) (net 12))
 (segment (start 122.682 112.522) (end 123.444 111.76) (width 0.3) (layer F.Cu) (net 12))
 (segment (start 123.444 111.76) (end 123.444 101.092) (width 0.3) (layer F.Cu) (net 12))
 (segment (start 122.682 100.33) (end 120.65 100.33) (width 0.3) (layer F.Cu) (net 12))
 (segment (start 123.444 101.092) (end 122.682 100.33) (width 0.3) (layer F.Cu) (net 12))
 (segment (start 110.87 103.87) (end 108.728 103.87) (width 0.3) (layer F.Cu) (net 13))
 (segment (start 108.728 103.87) (end 108.712 103.886) (width 0.3) (layer F.Cu) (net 13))
 (segment (start 108.712 103.886) (end 108.204 103.886) (width 0.3) (layer F.Cu) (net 13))
 (segment (start 108.204 103.886) (end 107.442 104.648) (width 0.3) (layer F.Cu) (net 13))
 (segment (start 107.442 104.648) (end 107.442 112.014) (width 0.3) (layer F.Cu) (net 13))
 (segment (start 107.442 112.014) (end 108.712 113.284) (width 0.3) (layer F.Cu) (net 13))
 (segment (start 108.712 113.284) (end 123.444 113.284) (width 0.3) (layer F.Cu) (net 13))
 (segment (start 123.444 113.284) (end 124.206 112.522) (width 0.3) (layer F.Cu) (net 13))
 (segment (start 124.206 112.522) (end 124.206 98.298) (width 0.3) (layer F.Cu) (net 13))
 (segment (start 123.698 97.79) (end 120.65 97.79) (width 0.3) (layer F.Cu) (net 13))
 (segment (start 124.206 98.298) (end 123.698 97.79) (width 0.3) (layer F.Cu) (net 13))
 (segment (start 94.79 97.79) (end 94.87 97.87) (width 0.5) (layer F.Cu) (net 7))
 (segment (start 88.9 97.79) (end 94.79 97.79) (width 0.3) (layer F.Cu) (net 7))
 (segment (start 125.222 96.012) (end 124.46 95.25) (width 0.3) (layer F.Cu) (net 14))
 (segment (start 125.222 113.284) (end 125.222 96.012) (width 0.3) (layer F.Cu) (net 14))
 (segment (start 124.46 114.046) (end 125.222 113.284) (width 0.3) (layer F.Cu) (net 14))
 (segment (start 107.442 114.046) (end 124.46 114.046) (width 0.3) (layer F.Cu) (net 14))
 (segment (start 124.46 95.25) (end 120.65 95.25) (width 0.3) (layer F.Cu) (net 14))
 (segment (start 106.426 108.458) (end 106.426 113.03) (width 0.3) (layer F.Cu) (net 14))
 (segment (start 106.426 113.03) (end 107.442 114.046) (width 0.3) (layer F.Cu) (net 14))
 (segment (start 105.838 107.87) (end 106.426 108.458) (width 0.3) (layer F.Cu) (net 14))
 (segment (start 94.87 107.87) (end 105.838 107.87) (width 0.3) (layer F.Cu) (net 14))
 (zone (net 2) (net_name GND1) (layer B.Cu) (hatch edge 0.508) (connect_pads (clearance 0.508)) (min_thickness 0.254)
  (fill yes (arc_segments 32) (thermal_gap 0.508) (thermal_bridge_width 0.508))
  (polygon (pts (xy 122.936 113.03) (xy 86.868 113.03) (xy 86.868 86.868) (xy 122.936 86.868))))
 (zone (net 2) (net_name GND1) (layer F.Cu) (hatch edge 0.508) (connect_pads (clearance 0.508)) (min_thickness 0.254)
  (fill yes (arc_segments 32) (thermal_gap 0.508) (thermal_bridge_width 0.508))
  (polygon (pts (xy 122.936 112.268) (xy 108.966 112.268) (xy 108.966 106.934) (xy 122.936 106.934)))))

